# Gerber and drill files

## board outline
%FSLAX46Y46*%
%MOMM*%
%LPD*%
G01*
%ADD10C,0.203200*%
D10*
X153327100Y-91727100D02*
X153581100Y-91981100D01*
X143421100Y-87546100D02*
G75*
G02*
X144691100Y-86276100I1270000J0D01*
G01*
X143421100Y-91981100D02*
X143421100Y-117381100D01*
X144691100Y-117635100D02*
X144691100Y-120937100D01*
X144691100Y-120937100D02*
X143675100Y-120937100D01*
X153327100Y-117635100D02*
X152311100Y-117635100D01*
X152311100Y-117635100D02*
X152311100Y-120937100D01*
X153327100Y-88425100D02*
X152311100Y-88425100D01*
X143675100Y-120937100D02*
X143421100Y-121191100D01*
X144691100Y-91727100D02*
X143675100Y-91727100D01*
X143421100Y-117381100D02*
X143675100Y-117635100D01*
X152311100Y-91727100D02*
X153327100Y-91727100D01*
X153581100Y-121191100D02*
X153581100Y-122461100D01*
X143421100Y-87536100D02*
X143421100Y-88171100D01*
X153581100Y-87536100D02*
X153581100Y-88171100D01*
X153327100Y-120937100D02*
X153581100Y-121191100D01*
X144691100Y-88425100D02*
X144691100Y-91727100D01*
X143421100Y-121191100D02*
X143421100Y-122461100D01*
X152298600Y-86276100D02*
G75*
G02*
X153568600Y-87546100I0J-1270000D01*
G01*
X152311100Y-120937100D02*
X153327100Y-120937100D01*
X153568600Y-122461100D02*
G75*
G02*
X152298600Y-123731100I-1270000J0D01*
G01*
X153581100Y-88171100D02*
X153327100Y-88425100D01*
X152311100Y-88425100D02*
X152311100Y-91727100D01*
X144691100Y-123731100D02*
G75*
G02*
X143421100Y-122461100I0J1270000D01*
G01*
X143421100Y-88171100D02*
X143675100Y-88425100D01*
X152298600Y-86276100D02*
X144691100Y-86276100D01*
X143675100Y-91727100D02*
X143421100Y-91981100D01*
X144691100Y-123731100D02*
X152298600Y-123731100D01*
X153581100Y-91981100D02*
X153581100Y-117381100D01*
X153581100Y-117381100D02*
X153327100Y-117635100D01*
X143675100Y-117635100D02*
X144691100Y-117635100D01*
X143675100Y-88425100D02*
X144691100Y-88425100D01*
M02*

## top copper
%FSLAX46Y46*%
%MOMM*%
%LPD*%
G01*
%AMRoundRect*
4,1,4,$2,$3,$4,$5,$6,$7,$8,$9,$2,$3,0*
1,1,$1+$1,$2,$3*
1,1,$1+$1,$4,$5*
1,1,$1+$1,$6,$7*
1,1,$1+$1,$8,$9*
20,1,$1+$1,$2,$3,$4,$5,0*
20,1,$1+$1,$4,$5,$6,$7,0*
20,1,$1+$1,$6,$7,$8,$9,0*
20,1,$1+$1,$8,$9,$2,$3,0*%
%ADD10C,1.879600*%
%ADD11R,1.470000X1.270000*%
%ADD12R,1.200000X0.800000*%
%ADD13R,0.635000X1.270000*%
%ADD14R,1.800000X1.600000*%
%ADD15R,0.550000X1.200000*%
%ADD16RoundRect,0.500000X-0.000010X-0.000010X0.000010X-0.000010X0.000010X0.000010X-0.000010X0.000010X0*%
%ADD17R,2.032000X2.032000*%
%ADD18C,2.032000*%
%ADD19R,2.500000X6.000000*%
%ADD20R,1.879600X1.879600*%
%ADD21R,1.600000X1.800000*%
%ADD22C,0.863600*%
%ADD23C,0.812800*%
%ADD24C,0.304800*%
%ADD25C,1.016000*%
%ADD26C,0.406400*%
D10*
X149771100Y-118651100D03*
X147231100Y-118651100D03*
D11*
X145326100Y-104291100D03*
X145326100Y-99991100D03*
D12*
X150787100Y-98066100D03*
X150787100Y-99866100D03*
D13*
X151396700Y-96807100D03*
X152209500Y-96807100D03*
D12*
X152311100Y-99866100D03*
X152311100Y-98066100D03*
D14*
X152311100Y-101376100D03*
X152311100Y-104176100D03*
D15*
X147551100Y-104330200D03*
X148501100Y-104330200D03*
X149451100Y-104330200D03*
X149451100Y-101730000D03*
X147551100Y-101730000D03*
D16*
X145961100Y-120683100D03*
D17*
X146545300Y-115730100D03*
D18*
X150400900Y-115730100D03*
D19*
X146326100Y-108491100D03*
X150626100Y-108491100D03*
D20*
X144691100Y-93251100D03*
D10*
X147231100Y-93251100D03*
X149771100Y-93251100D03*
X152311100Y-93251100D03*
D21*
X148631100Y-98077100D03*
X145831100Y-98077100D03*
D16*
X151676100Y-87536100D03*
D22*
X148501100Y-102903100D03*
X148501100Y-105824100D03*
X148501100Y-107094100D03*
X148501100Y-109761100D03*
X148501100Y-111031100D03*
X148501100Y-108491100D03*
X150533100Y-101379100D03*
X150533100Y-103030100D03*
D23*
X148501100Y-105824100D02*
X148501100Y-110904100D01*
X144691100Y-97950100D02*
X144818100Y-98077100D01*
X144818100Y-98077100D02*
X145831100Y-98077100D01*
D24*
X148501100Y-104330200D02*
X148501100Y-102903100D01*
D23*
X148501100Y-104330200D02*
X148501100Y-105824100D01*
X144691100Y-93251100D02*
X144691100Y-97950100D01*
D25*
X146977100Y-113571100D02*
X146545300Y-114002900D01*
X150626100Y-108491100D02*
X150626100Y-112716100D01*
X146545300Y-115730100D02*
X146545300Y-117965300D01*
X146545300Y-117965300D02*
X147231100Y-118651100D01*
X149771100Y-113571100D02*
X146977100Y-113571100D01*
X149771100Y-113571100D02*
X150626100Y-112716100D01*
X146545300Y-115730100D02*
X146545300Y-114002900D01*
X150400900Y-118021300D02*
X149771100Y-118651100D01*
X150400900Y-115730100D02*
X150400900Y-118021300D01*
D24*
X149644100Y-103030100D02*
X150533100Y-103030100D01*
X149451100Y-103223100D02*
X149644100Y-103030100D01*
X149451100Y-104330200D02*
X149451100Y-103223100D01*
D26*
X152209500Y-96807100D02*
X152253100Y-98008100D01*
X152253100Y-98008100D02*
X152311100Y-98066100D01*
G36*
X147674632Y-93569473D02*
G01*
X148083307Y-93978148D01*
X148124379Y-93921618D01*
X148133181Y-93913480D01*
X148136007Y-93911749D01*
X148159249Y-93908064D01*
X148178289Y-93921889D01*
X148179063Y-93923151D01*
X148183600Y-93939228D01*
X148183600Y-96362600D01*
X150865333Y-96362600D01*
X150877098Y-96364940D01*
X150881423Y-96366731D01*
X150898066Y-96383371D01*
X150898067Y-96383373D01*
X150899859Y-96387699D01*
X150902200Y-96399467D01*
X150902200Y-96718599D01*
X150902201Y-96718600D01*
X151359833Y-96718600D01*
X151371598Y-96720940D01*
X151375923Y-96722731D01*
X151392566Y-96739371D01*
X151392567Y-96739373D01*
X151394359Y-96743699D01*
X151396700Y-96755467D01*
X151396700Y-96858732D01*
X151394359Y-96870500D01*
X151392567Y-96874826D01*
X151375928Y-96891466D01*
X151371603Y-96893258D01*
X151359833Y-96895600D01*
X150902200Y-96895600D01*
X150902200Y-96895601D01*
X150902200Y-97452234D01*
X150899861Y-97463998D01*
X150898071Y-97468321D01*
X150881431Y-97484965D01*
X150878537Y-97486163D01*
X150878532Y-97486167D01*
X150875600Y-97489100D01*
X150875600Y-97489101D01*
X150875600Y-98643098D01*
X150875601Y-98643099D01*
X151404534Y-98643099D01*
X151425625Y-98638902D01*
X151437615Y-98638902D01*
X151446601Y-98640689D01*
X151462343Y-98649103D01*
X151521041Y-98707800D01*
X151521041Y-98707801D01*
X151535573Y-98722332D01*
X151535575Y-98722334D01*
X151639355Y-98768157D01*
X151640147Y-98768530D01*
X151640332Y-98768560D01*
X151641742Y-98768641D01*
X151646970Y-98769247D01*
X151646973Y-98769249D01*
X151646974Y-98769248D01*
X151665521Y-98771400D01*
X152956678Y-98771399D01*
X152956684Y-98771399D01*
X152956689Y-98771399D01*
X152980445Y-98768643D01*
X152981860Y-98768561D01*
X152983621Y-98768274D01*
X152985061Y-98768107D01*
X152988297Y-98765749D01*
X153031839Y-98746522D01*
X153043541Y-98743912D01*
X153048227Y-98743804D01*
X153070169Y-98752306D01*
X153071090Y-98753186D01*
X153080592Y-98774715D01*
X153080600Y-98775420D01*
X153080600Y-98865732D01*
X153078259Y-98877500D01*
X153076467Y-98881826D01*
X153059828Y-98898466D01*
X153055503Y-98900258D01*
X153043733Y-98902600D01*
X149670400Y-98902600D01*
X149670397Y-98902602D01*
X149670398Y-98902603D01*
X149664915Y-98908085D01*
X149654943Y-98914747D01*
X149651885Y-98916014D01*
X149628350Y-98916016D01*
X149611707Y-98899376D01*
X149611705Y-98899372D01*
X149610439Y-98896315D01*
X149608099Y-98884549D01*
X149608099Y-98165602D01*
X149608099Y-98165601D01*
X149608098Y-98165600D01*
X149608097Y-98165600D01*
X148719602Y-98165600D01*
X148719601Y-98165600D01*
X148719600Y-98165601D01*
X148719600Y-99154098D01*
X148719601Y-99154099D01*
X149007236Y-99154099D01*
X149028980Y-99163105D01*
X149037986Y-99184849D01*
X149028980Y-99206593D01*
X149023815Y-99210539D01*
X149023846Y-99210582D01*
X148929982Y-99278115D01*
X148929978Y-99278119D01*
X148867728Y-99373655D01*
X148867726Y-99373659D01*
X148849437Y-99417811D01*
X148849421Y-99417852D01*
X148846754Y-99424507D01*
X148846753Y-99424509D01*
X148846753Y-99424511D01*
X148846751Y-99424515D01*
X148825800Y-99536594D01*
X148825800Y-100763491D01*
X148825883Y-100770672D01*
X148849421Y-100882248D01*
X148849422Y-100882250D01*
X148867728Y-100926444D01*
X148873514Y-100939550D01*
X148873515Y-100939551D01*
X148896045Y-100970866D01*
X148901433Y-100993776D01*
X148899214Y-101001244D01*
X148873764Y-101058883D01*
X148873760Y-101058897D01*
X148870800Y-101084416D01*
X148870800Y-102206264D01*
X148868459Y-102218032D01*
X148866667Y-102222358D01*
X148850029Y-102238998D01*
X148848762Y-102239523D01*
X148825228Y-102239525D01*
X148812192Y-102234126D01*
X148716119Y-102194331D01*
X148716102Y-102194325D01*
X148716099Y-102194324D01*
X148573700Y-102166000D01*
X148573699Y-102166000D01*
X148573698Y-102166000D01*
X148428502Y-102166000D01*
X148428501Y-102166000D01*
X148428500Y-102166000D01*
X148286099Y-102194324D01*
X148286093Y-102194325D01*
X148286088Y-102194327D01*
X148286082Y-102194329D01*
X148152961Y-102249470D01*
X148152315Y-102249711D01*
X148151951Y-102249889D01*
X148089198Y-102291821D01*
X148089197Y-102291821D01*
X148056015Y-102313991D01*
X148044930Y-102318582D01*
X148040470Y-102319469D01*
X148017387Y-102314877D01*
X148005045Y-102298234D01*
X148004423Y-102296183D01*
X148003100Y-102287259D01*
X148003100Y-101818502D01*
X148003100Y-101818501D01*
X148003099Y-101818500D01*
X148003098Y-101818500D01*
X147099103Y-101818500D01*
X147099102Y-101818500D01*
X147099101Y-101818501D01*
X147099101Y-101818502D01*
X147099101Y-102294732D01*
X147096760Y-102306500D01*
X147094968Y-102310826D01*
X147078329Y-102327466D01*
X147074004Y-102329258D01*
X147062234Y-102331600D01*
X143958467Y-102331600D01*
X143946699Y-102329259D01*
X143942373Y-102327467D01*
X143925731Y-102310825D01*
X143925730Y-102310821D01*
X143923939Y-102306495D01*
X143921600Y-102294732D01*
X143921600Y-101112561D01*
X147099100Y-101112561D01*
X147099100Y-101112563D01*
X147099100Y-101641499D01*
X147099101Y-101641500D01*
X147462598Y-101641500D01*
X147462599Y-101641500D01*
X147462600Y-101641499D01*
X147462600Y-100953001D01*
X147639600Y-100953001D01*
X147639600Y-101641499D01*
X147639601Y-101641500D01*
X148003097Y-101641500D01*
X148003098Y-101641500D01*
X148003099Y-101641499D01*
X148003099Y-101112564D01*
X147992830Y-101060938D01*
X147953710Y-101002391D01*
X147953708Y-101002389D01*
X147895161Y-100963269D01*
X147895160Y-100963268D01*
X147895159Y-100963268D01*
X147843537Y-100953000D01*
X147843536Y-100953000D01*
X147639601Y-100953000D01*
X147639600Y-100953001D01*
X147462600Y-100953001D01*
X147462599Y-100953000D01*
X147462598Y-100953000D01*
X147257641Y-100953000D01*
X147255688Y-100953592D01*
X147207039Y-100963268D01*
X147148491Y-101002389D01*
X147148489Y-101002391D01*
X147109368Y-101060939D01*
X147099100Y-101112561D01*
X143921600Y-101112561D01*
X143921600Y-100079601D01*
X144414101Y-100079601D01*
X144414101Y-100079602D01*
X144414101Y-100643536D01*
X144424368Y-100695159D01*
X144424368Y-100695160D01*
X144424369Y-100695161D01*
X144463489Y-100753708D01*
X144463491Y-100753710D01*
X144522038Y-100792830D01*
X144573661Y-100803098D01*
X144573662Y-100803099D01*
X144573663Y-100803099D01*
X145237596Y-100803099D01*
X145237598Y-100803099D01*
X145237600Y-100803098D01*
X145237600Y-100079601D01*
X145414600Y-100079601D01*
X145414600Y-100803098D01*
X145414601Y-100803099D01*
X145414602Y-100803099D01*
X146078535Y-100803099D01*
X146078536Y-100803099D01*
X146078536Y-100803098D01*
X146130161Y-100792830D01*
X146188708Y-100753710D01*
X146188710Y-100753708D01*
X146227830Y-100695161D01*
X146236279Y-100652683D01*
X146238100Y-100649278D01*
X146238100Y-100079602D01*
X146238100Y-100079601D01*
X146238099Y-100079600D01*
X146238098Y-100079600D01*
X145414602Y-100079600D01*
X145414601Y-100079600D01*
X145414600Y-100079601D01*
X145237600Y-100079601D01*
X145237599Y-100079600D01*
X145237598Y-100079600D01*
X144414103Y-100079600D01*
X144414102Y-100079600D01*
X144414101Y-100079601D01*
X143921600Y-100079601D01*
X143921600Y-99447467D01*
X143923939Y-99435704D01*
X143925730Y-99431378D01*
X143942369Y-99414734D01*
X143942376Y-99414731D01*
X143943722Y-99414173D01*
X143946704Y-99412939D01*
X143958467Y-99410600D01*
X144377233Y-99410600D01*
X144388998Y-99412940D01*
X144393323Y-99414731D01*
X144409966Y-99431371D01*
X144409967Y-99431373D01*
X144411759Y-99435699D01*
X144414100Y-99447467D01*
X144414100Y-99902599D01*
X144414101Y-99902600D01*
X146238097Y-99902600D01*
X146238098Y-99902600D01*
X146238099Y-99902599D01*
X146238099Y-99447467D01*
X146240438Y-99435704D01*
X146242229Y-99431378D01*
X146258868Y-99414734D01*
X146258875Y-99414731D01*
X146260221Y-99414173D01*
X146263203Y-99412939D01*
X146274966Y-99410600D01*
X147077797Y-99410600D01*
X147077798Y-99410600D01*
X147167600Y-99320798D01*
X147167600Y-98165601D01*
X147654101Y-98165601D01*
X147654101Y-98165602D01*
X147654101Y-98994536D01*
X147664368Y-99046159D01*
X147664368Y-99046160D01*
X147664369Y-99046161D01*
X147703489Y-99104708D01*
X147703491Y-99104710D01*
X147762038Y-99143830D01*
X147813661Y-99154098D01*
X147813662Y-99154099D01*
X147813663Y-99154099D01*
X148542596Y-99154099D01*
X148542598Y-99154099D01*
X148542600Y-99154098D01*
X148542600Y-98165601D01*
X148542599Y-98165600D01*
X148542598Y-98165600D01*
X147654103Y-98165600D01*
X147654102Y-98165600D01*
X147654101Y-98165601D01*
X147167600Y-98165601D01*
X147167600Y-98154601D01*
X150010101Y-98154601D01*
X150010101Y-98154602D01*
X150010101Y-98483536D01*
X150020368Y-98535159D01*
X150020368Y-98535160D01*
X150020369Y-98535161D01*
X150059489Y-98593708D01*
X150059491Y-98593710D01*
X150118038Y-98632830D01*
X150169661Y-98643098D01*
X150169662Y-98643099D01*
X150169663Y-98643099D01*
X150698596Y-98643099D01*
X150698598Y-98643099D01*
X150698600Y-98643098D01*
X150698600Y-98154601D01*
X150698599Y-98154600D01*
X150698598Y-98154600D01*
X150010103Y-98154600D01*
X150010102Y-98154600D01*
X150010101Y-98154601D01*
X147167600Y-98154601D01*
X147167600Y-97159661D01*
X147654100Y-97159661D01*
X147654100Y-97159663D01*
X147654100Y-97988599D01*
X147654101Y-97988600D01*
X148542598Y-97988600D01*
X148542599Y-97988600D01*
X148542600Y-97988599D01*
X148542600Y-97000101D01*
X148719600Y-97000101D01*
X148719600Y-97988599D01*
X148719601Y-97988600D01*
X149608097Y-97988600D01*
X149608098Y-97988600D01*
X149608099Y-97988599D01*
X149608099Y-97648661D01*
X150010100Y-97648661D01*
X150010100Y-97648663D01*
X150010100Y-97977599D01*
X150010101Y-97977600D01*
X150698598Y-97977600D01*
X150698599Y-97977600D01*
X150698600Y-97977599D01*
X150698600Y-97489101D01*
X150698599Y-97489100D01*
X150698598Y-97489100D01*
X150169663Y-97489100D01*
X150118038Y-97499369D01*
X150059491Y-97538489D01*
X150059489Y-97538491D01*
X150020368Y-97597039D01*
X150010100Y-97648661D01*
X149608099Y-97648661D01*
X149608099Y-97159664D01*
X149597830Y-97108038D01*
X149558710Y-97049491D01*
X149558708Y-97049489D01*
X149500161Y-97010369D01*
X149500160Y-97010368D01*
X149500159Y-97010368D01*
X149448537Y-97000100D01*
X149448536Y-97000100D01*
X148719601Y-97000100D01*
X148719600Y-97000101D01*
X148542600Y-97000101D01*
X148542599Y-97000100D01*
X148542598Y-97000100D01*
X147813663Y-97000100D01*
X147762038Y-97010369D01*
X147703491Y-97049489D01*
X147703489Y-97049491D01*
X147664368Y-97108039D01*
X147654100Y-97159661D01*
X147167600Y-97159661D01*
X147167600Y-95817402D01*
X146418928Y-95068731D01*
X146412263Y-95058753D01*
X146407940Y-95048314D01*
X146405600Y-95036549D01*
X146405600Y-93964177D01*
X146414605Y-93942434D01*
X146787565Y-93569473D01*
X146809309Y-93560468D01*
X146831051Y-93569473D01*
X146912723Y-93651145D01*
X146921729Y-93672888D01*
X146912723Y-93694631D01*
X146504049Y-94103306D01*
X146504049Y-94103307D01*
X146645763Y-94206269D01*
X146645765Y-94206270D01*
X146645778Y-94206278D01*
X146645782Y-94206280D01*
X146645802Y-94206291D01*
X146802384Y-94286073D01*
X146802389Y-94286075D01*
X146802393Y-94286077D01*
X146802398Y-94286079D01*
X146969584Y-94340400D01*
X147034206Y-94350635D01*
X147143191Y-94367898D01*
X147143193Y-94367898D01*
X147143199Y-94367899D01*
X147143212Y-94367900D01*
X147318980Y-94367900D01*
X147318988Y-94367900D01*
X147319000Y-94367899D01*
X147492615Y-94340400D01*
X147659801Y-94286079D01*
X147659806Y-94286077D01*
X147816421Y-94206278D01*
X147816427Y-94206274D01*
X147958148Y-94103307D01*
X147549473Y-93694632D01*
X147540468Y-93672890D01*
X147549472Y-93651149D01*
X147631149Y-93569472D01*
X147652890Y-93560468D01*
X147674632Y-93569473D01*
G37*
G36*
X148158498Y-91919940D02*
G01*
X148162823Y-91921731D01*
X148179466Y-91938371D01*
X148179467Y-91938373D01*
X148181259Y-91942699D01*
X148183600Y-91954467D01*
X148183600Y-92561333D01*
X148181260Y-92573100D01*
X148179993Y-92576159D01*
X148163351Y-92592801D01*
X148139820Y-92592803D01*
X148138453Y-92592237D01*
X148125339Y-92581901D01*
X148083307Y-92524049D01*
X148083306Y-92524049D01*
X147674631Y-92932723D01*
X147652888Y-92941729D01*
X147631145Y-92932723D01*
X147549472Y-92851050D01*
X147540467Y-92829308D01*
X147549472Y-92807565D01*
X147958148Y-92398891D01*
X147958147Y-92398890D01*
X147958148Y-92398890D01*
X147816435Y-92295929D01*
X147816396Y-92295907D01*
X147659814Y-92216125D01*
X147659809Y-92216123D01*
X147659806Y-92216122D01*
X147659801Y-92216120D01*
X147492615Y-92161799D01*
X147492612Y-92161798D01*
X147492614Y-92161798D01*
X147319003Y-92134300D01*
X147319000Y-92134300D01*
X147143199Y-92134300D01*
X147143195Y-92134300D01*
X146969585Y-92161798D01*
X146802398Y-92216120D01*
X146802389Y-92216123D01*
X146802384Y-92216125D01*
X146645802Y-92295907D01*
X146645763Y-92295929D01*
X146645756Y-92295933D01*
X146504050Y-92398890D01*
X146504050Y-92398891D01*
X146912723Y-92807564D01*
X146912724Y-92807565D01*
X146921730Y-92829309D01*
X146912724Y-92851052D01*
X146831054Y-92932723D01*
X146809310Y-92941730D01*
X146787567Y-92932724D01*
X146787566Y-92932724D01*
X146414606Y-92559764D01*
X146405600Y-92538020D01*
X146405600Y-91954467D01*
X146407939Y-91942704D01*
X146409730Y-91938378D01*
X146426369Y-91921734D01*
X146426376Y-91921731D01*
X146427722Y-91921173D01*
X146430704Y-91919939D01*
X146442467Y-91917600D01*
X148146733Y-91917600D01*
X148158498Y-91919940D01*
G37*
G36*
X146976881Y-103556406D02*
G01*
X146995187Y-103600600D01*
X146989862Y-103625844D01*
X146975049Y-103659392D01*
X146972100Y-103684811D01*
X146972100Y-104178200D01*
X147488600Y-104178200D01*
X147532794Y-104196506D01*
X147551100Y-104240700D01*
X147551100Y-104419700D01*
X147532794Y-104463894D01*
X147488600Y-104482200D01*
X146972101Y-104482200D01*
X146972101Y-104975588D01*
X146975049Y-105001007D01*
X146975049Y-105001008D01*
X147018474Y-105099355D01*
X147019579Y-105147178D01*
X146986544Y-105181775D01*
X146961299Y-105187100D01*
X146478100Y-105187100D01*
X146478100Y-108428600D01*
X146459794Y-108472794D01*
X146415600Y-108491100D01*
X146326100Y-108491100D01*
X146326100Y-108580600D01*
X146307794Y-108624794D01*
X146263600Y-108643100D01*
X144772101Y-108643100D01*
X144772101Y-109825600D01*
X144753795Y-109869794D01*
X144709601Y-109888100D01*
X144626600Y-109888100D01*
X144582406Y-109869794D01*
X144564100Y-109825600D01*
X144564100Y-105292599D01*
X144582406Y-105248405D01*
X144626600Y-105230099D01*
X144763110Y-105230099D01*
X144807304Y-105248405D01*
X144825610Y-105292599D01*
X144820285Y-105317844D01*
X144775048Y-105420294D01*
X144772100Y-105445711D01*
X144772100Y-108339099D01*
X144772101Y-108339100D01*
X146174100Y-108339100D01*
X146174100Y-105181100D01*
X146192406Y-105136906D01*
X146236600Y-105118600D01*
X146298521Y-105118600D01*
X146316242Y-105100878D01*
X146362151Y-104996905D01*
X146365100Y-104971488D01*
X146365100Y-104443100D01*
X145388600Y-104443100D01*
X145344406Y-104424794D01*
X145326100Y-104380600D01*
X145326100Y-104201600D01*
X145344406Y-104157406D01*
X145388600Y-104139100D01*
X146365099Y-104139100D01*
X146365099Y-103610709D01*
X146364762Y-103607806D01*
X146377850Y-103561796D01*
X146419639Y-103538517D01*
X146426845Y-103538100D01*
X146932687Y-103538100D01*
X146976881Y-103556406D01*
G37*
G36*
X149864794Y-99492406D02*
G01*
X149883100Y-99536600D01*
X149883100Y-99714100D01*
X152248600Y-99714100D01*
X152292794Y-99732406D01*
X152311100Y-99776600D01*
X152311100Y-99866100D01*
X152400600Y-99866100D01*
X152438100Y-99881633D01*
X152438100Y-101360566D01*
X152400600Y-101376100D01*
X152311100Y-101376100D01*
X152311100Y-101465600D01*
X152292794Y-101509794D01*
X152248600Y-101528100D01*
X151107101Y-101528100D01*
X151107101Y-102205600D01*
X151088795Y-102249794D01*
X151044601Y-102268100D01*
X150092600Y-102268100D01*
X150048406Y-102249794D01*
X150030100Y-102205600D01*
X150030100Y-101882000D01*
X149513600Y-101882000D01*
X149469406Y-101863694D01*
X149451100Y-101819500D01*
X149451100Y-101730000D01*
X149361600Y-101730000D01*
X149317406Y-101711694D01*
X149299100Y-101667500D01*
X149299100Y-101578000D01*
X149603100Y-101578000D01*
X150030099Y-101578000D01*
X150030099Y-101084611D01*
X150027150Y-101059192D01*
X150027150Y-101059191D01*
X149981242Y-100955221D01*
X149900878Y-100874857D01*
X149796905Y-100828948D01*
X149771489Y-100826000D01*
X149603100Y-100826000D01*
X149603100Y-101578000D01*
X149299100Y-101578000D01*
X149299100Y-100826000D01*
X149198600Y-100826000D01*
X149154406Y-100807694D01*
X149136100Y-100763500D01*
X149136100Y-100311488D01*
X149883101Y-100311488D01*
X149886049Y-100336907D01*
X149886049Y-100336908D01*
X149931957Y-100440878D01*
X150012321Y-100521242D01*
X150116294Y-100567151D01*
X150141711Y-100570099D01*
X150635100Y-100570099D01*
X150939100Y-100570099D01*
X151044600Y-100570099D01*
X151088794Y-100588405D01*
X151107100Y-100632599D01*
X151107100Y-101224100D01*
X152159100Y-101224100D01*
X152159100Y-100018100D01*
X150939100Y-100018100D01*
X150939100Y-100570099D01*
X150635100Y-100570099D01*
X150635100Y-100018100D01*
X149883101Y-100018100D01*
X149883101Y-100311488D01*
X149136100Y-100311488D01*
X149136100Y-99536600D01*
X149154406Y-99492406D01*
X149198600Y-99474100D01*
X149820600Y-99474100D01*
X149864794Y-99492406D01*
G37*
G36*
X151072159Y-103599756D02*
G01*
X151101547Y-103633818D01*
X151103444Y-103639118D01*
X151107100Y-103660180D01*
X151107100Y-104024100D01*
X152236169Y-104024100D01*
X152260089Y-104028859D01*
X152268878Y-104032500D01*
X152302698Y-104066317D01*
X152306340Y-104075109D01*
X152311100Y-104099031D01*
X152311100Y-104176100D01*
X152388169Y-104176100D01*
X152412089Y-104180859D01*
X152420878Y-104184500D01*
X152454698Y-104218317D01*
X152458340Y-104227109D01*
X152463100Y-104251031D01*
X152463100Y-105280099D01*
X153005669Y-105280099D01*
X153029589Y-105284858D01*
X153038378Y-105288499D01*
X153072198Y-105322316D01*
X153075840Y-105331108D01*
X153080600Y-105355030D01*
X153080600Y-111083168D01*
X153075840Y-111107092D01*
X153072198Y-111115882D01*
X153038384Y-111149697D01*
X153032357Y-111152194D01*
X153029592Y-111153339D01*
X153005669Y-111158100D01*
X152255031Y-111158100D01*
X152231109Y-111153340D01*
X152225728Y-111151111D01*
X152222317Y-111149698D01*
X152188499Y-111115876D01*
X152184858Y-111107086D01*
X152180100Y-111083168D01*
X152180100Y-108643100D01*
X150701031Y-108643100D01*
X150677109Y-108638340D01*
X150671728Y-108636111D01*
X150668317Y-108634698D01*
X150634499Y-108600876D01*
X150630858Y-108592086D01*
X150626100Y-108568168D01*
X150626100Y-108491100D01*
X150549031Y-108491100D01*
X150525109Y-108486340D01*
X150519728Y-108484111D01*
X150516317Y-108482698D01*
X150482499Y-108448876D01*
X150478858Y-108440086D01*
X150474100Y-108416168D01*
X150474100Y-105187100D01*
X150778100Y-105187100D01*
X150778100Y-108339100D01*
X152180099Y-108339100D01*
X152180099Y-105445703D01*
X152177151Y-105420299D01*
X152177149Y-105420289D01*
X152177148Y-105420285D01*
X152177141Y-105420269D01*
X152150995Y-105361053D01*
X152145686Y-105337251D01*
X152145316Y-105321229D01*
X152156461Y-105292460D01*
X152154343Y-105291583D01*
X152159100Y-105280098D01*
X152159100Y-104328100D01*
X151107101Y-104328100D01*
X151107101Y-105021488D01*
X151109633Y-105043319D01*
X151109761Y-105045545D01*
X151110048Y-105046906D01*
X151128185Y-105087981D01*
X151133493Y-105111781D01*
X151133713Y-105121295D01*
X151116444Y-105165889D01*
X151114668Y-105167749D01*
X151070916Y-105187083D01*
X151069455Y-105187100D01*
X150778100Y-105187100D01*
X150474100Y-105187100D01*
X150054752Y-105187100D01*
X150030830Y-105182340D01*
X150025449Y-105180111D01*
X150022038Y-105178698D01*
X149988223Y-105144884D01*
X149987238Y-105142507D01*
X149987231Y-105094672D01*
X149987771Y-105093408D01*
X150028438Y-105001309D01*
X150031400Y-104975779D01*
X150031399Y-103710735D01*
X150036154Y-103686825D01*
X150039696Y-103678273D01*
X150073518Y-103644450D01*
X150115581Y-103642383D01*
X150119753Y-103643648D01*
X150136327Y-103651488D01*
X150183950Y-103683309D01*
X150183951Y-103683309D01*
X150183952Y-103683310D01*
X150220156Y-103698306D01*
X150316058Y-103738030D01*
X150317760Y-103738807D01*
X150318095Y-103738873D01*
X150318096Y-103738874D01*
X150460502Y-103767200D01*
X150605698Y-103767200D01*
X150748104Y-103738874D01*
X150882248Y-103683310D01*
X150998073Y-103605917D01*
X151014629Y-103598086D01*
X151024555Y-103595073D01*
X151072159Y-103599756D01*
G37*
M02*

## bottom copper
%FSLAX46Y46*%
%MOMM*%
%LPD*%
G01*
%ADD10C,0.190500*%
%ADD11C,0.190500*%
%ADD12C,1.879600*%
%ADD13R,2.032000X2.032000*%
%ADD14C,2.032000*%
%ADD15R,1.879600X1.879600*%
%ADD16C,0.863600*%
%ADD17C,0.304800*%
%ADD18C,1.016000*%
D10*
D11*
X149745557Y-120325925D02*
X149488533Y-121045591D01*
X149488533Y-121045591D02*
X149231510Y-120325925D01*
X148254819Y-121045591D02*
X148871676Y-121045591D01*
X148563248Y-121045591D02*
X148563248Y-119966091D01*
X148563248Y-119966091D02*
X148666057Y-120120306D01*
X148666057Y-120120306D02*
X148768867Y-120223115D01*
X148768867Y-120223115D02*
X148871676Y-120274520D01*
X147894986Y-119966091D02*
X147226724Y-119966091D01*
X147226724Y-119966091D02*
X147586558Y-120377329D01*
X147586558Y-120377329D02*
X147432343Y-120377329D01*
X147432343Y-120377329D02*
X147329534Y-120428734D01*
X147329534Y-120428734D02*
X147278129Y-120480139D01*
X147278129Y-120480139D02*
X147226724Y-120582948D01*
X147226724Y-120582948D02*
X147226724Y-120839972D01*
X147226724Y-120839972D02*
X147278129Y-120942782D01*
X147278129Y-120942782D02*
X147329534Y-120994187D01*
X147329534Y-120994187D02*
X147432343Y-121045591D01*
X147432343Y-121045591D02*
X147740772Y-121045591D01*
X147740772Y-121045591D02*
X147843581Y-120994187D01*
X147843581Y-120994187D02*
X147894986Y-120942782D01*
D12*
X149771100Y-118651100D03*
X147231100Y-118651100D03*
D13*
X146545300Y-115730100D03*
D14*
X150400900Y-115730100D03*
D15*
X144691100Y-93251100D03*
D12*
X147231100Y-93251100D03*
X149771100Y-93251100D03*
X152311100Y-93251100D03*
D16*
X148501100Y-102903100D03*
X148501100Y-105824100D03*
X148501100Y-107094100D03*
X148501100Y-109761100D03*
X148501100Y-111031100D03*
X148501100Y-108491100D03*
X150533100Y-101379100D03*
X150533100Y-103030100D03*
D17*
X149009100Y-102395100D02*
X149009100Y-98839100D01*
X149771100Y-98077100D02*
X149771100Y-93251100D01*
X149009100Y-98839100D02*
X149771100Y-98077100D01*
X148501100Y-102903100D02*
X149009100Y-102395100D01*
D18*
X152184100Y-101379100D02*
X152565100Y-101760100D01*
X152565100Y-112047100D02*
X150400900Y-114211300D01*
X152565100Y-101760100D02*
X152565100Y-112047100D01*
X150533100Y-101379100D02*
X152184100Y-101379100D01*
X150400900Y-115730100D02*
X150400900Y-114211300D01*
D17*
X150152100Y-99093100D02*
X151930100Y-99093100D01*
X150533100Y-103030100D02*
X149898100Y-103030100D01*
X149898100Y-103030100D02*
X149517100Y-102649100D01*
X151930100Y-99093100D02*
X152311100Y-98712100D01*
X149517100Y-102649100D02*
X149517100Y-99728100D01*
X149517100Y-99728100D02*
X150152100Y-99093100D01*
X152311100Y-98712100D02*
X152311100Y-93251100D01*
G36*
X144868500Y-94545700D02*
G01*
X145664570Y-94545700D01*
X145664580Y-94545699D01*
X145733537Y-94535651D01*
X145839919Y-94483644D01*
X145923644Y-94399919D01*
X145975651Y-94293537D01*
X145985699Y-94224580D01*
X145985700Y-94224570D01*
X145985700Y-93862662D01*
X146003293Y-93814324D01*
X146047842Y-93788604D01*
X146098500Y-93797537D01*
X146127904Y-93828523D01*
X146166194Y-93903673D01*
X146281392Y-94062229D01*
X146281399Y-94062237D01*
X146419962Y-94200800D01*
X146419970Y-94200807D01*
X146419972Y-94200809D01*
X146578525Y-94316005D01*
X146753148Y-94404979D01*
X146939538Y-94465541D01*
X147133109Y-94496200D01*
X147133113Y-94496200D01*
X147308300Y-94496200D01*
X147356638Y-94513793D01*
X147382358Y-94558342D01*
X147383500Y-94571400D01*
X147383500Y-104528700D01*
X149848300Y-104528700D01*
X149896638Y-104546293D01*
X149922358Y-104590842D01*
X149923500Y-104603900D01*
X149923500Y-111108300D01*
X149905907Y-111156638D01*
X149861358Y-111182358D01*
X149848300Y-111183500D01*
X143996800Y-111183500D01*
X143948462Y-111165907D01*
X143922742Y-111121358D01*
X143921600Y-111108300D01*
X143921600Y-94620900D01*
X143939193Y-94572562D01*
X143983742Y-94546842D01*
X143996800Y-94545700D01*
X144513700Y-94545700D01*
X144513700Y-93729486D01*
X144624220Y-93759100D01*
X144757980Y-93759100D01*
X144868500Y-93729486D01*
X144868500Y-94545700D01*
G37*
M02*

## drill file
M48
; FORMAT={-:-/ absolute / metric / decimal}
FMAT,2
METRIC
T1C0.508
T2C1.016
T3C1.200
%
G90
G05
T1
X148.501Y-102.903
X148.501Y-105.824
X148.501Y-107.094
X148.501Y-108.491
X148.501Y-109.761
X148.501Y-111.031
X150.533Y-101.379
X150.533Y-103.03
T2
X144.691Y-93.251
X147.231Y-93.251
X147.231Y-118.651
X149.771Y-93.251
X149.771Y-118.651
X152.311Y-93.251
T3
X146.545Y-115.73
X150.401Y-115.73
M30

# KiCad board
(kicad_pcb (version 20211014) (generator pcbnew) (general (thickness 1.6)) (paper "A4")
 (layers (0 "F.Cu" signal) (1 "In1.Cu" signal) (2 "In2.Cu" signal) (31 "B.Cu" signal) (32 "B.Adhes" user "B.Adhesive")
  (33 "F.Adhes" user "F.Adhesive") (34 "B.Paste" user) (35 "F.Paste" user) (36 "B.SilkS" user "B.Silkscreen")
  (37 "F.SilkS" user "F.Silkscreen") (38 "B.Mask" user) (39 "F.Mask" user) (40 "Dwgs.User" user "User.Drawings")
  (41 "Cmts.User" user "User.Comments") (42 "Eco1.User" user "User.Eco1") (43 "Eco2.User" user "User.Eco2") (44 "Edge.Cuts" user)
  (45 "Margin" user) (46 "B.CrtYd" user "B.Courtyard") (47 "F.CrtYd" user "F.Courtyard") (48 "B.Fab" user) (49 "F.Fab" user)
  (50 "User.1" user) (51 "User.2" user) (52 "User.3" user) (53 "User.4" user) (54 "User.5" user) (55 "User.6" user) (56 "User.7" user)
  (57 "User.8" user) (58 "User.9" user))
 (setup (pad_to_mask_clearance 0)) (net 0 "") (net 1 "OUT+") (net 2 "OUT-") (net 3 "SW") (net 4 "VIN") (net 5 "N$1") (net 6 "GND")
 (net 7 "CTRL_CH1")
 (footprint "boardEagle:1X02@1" (layer "F.Cu") (at 149.7711 118.6511 180)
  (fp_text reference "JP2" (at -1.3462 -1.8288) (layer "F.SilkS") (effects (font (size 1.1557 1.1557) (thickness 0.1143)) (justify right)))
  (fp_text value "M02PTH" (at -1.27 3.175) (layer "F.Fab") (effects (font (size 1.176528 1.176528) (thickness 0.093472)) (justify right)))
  (pad "1" thru_hole circle (at 0 0 270) (size 1.8796 1.8796) (drill 1.016) (layers *.Cu *.Mask) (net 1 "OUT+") (solder_mask_margin 0.1016))
  (pad "2" thru_hole circle (at 2.54 0 270) (size 1.8796 1.8796) (drill 1.016) (layers *.Cu *.Mask) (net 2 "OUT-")
   (solder_mask_margin 0.1016)))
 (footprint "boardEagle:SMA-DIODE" (layer "F.Cu") (at 145.3261 102.1411 90)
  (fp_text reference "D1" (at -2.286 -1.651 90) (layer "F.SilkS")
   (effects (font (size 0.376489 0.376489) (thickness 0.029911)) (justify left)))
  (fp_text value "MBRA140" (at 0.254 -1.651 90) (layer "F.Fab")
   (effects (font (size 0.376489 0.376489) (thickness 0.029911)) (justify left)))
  (pad "A" smd rect (at -2.15 0 270) (size 1.27 1.47) (layers "F.Cu" "F.Paste" "F.Mask") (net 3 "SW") (solder_mask_margin 0.1016))
  (pad "C" smd rect (at 2.15 0 90) (size 1.27 1.47) (layers "F.Cu" "F.Paste" "F.Mask") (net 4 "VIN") (solder_mask_margin 0.1016)))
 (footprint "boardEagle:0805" (layer "F.Cu") (at 150.7871 98.9661 -90)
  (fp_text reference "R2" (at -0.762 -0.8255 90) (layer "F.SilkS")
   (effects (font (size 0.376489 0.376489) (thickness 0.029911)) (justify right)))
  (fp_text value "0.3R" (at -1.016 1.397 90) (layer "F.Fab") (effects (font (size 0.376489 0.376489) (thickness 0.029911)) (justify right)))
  (pad "1" smd rect (at -0.9 0 270) (size 0.8 1.2) (layers "F.Cu" "F.Paste" "F.Mask") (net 4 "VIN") (solder_mask_margin 0.1016))
  (pad "2" smd rect (at 0.9 0 270) (size 0.8 1.2) (layers "F.Cu" "F.Paste" "F.Mask") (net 1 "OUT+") (solder_mask_margin 0.1016)))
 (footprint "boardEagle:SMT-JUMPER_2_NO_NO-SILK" (layer "F.Cu") (at 151.8031 96.8071)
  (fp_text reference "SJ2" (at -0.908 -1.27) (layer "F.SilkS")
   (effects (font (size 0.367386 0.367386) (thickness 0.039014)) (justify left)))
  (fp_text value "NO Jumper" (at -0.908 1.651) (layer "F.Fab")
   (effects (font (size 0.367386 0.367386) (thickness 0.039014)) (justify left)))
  (pad "1" smd rect (at -0.4064 0) (size 0.635 1.27) (layers "F.Cu" "F.Mask") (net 4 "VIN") (solder_mask_margin 0.1016))
  (pad "2" smd rect (at 0.4064 0) (size 0.635 1.27) (layers "F.Cu" "F.Mask") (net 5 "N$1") (solder_mask_margin 0.1016)))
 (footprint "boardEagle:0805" (layer "F.Cu") (at 152.3111 98.9661 90)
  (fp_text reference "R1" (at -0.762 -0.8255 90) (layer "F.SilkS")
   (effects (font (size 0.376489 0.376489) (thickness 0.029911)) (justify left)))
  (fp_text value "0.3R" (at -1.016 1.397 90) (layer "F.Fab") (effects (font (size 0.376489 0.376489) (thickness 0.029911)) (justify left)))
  (pad "1" smd rect (at -0.9 0 90) (size 0.8 1.2) (layers "F.Cu" "F.Paste" "F.Mask") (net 1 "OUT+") (solder_mask_margin 0.1016))
  (pad "2" smd rect (at 0.9 0 90) (size 0.8 1.2) (layers "F.Cu" "F.Paste" "F.Mask") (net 5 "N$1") (solder_mask_margin 0.1016)))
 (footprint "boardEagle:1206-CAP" (layer "F.Cu") (at 152.3111 102.7761 -90)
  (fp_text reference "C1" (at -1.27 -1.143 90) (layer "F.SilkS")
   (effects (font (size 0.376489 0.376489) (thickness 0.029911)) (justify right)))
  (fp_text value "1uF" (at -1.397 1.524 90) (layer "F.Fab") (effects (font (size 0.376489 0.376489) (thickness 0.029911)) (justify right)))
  (pad "1" smd rect (at -1.4 0 270) (size 1.6 1.8) (layers "F.Cu" "F.Paste" "F.Mask") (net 1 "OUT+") (solder_mask_margin 0.1016))
  (pad "2" smd rect (at 1.4 0 270) (size 1.6 1.8) (layers "F.Cu" "F.Paste" "F.Mask") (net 2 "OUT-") (solder_mask_margin 0.1016)))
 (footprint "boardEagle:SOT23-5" (layer "F.Cu") (at 148.5011 103.0301)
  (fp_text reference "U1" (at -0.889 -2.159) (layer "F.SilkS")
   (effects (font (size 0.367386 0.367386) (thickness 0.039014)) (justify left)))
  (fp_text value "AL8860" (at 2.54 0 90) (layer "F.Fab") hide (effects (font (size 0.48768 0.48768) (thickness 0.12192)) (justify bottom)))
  (pad "1" smd rect (at -0.95 1.3001) (size 0.55 1.2) (layers "F.Cu" "F.Paste" "F.Mask") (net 3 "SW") (solder_mask_margin 0.1016))
  (pad "2" smd rect (at 0 1.3001) (size 0.55 1.2) (layers "F.Cu" "F.Paste" "F.Mask") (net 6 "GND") (solder_mask_margin 0.1016))
  (pad "3" smd rect (at 0.95 1.3001) (size 0.55 1.2) (layers "F.Cu" "F.Paste" "F.Mask") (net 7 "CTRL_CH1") (solder_mask_margin 0.1016))
  (pad "4" smd rect (at 0.95 -1.3001) (size 0.55 1.2) (layers "F.Cu" "F.Paste" "F.Mask") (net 1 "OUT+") (solder_mask_margin 0.1016))
  (pad "5" smd rect (at -0.95 -1.3001) (size 0.55 1.2) (layers "F.Cu" "F.Paste" "F.Mask") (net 4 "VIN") (solder_mask_margin 0.1016)))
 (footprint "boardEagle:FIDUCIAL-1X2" (layer "F.Cu") (at 145.9611 120.6831)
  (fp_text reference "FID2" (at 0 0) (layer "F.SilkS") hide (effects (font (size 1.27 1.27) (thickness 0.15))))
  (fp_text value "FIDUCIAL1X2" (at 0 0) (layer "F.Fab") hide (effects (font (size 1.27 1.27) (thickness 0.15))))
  (pad "1" smd roundrect (at 0 0) (size 1 1) (layers "F.Cu" "F.Mask") (roundrect_rratio 0.5) (solder_mask_margin 0.1016)))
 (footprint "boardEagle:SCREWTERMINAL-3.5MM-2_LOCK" (layer "F.Cu") (at 146.7231 115.7301)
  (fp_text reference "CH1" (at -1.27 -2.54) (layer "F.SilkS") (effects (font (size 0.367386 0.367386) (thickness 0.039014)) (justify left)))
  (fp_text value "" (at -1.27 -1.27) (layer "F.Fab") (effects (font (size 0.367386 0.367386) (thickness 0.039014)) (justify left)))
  (pad "1" thru_hole rect (at -0.1778 0) (size 2.032 2.032) (drill 1.2) (layers *.Cu *.Mask) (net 2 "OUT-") (solder_mask_margin 0.1016))
  (pad "2" thru_hole circle (at 3.6778 0) (size 2.032 2.032) (drill 1.2) (layers *.Cu *.Mask) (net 1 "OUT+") (solder_mask_margin 0.1016)))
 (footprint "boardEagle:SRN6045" (layer "F.Cu") (at 148.5011 108.4911)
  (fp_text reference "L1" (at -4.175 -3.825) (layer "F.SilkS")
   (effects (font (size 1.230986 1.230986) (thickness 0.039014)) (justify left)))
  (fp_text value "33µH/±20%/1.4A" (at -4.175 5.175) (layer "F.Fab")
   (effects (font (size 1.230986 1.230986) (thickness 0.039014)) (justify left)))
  (pad "1" smd rect (at -2.175 0 90) (size 6 2.5) (layers "F.Cu" "F.Paste" "F.Mask") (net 3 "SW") (solder_mask_margin 0.1016))
  (pad "2" smd rect (at 2.125 0 90) (size 6 2.5) (layers "F.Cu" "F.Paste" "F.Mask") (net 2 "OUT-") (solder_mask_margin 0.1016)))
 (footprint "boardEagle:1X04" (layer "F.Cu") (at 144.6911 93.2511)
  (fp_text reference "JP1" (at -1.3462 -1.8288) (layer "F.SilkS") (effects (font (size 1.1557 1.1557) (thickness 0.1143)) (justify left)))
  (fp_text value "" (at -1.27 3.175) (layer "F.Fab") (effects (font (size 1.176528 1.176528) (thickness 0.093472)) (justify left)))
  (pad "1" thru_hole rect (at 0 0 90) (size 1.8796 1.8796) (drill 1.016) (layers *.Cu *.Mask) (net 6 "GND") (solder_mask_margin 0.1016))
  (pad "2" thru_hole circle (at 2.54 0 90) (size 1.8796 1.8796) (drill 1.016) (layers *.Cu *.Mask) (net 4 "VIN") (solder_mask_margin 0.1016))
  (pad "3" thru_hole circle (at 5.08 0 90) (size 1.8796 1.8796) (drill 1.016) (layers *.Cu *.Mask) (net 6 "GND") (solder_mask_margin 0.1016))
  (pad "4" thru_hole circle (at 7.62 0 90) (size 1.8796 1.8796) (drill 1.016) (layers *.Cu *.Mask) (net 7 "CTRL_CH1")
   (solder_mask_margin 0.1016)))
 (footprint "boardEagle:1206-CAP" (layer "F.Cu") (at 147.2311 98.0771 180)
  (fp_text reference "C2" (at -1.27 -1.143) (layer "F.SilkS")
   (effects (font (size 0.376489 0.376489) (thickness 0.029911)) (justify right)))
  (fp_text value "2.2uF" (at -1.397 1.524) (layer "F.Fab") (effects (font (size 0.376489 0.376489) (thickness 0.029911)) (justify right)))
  (pad "1" smd rect (at -1.4 0 180) (size 1.6 1.8) (layers "F.Cu" "F.Paste" "F.Mask") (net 4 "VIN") (solder_mask_margin 0.1016))
  (pad "2" smd rect (at 1.4 0 180) (size 1.6 1.8) (layers "F.Cu" "F.Paste" "F.Mask") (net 6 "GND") (solder_mask_margin 0.1016)))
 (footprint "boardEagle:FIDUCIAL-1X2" (layer "F.Cu") (at 151.6761 87.5361)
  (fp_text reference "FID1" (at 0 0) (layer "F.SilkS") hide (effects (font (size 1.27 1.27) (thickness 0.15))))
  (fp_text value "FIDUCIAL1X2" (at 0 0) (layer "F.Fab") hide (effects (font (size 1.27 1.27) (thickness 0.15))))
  (pad "1" smd roundrect (at 0 0) (size 1 1) (layers "F.Cu" "F.Mask") (roundrect_rratio 0.5) (solder_mask_margin 0.1016)))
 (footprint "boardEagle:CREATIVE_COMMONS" (layer "F.Cu") (at 154.8511 145.3211)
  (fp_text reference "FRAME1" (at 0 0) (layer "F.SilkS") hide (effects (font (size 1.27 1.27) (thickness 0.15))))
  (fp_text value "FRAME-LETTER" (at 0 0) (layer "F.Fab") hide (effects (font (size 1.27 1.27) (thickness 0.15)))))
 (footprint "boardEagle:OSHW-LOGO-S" (layer "B.Cu") (at 145.4531 98.7121 -90)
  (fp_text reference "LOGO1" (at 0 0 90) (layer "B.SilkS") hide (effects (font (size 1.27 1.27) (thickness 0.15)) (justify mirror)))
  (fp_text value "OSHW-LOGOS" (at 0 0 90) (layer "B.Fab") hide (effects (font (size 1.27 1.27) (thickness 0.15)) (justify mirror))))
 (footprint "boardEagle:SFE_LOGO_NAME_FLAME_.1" (layer "B.Cu") (at 153.2001 100.6171 -90)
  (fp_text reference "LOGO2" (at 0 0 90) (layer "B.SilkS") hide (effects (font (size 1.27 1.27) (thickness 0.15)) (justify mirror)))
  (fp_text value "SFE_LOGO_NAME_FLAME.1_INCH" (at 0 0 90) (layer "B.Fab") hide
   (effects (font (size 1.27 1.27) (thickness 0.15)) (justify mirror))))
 (gr_line (start 153.3271 91.7271) (end 153.5811 91.9811) (layer "Edge.Cuts") (width 0.2032))
 (gr_arc (start 143.4211 87.5461) (mid 143.793074 86.648074) (end 144.6911 86.2761) (layer "Edge.Cuts") (width 0.2032))
 (gr_line (start 143.4211 91.9811) (end 143.4211 117.3811) (layer "Edge.Cuts") (width 0.2032))
 (gr_line (start 144.6911 117.6351) (end 144.6911 120.9371) (layer "Edge.Cuts") (width 0.2032))
 (gr_line (start 144.6911 120.9371) (end 143.6751 120.9371) (layer "Edge.Cuts") (width 0.2032))
 (gr_line (start 153.3271 117.6351) (end 152.3111 117.6351) (layer "Edge.Cuts") (width 0.2032))
 (gr_line (start 152.3111 117.6351) (end 152.3111 120.9371) (layer "Edge.Cuts") (width 0.2032))
 (gr_line (start 153.3271 88.4251) (end 152.3111 88.4251) (layer "Edge.Cuts") (width 0.2032))
 (gr_line (start 143.6751 120.9371) (end 143.4211 121.1911) (layer "Edge.Cuts") (width 0.2032))
 (gr_line (start 144.6911 91.7271) (end 143.6751 91.7271) (layer "Edge.Cuts") (width 0.2032))
 (gr_line (start 143.4211 117.3811) (end 143.6751 117.6351) (layer "Edge.Cuts") (width 0.2032))
 (gr_line (start 152.3111 91.7271) (end 153.3271 91.7271) (layer "Edge.Cuts") (width 0.2032))
 (gr_line (start 153.5811 121.1911) (end 153.5811 122.4611) (layer "Edge.Cuts") (width 0.2032))
 (gr_line (start 143.4211 87.5361) (end 143.4211 88.1711) (layer "Edge.Cuts") (width 0.2032))
 (gr_line (start 153.5811 87.5361) (end 153.5811 88.1711) (layer "Edge.Cuts") (width 0.2032))
 (gr_line (start 153.3271 120.9371) (end 153.5811 121.1911) (layer "Edge.Cuts") (width 0.2032))
 (gr_line (start 144.6911 88.4251) (end 144.6911 91.7271) (layer "Edge.Cuts") (width 0.2032))
 (gr_line (start 143.4211 121.1911) (end 143.4211 122.4611) (layer "Edge.Cuts") (width 0.2032))
 (gr_arc (start 152.2986 86.2761) (mid 153.196626 86.648074) (end 153.5686 87.5461) (layer "Edge.Cuts") (width 0.2032))
 (gr_line (start 152.3111 120.9371) (end 153.3271 120.9371) (layer "Edge.Cuts") (width 0.2032))
 (gr_arc (start 153.5686 122.4611) (mid 153.196626 123.359126) (end 152.2986 123.7311) (layer "Edge.Cuts") (width 0.2032))
 (gr_line (start 153.5811 88.1711) (end 153.3271 88.4251) (layer "Edge.Cuts") (width 0.2032))
 (gr_line (start 152.3111 88.4251) (end 152.3111 91.7271) (layer "Edge.Cuts") (width 0.2032))
 (gr_arc (start 144.6911 123.7311) (mid 143.793074 123.359126) (end 143.4211 122.4611) (layer "Edge.Cuts") (width 0.2032))
 (gr_line (start 143.4211 88.1711) (end 143.6751 88.4251) (layer "Edge.Cuts") (width 0.2032))
 (gr_line (start 152.2986 86.2761) (end 144.6911 86.2761) (layer "Edge.Cuts") (width 0.2032))
 (gr_line (start 143.6751 91.7271) (end 143.4211 91.9811) (layer "Edge.Cuts") (width 0.2032))
 (gr_line (start 144.6911 123.7311) (end 152.2986 123.7311) (layer "Edge.Cuts") (width 0.2032))
 (gr_line (start 153.5811 91.9811) (end 153.5811 117.3811) (layer "Edge.Cuts") (width 0.2032))
 (gr_line (start 153.5811 117.3811) (end 153.3271 117.6351) (layer "Edge.Cuts") (width 0.2032))
 (gr_line (start 143.6751 117.6351) (end 144.6911 117.6351) (layer "Edge.Cuts") (width 0.2032))
 (gr_line (start 143.6751 88.4251) (end 144.6911 88.4251) (layer "Edge.Cuts") (width 0.2032))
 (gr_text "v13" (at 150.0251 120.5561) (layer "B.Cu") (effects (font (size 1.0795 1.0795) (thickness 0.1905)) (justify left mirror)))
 (segment (start 148.5011 105.8241) (end 148.5011 110.9041) (width 0.8128) (layer "F.Cu") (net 6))
 (segment (start 144.6911 97.9501) (end 144.8181 98.0771) (width 0.8128) (layer "F.Cu") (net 6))
 (segment (start 144.8181 98.0771) (end 145.8311 98.0771) (width 0.8128) (layer "F.Cu") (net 6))
 (segment (start 148.5011 104.3302) (end 148.5011 102.9031) (width 0.3048) (layer "F.Cu") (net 6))
 (segment (start 148.5011 104.3302) (end 148.5011 105.8241) (width 0.8128) (layer "F.Cu") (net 6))
 (segment (start 144.6911 93.2511) (end 144.6911 97.9501) (width 0.8128) (layer "F.Cu") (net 6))
 (via (at 148.5011 102.9031) (size 0.8636) (drill 0.508) (layers "F.Cu" "B.Cu") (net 6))
 (via (at 148.5011 105.8241) (size 0.8636) (drill 0.508) (layers "F.Cu" "B.Cu") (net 6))
 (via (at 148.5011 107.0941) (size 0.8636) (drill 0.508) (layers "F.Cu" "B.Cu") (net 6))
 (via (at 148.5011 109.7611) (size 0.8636) (drill 0.508) (layers "F.Cu" "B.Cu") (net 6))
 (via (at 148.5011 111.0311) (size 0.8636) (drill 0.508) (layers "F.Cu" "B.Cu") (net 6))
 (via (at 148.5011 108.4911) (size 0.8636) (drill 0.508) (layers "F.Cu" "B.Cu") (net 6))
 (segment (start 149.0091 102.3951) (end 149.0091 98.8391) (width 0.3048) (layer "B.Cu") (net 6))
 (segment (start 149.7711 98.0771) (end 149.7711 93.2511) (width 0.3048) (layer "B.Cu") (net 6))
 (segment (start 149.0091 98.8391) (end 149.7711 98.0771) (width 0.3048) (layer "B.Cu") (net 6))
 (segment (start 148.5011 102.9031) (end 149.0091 102.3951) (width 0.3048) (layer "B.Cu") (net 6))
 (segment (start 146.9771 113.5711) (end 146.5453 114.0029) (width 1.016) (layer "F.Cu") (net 2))
 (segment (start 150.6261 108.4911) (end 150.6261 112.7161) (width 1.016) (layer "F.Cu") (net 2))
 (segment (start 146.5453 115.7301) (end 146.5453 117.9653) (width 1.016) (layer "F.Cu") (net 2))
 (segment (start 146.5453 117.9653) (end 147.2311 118.6511) (width 1.016) (layer "F.Cu") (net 2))
 (segment (start 149.7711 113.5711) (end 146.9771 113.5711) (width 1.016) (layer "F.Cu") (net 2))
 (segment (start 149.7711 113.5711) (end 150.6261 112.7161) (width 1.016) (layer "F.Cu") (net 2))
 (segment (start 146.5453 115.7301) (end 146.5453 114.0029) (width 1.016) (layer "F.Cu") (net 2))
 (segment (start 150.4009 118.0213) (end 149.7711 118.6511) (width 1.016) (layer "F.Cu") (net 1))
 (segment (start 150.4009 115.7301) (end 150.4009 118.0213) (width 1.016) (layer "F.Cu") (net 1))
 (via (at 150.5331 101.3791) (size 0.8636) (drill 0.508) (layers "F.Cu" "B.Cu") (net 1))
 (segment (start 152.1841 101.3791) (end 152.5651 101.7601) (width 1.016) (layer "B.Cu") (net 1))
 (segment (start 152.5651 112.0471) (end 150.4009 114.2113) (width 1.016) (layer "B.Cu") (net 1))
 (segment (start 152.5651 101.7601) (end 152.5651 112.0471) (width 1.016) (layer "B.Cu") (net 1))
 (segment (start 150.5331 101.3791) (end 152.1841 101.3791) (width 1.016) (layer "B.Cu") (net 1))
 (segment (start 150.4009 115.7301) (end 150.4009 114.2113) (width 1.016) (layer "B.Cu") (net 1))
 (segment (start 149.6441 103.0301) (end 150.5331 103.0301) (width 0.3048) (layer "F.Cu") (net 7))
 (segment (start 149.4511 103.2231) (end 149.6441 103.0301) (width 0.3048) (layer "F.Cu") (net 7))
 (segment (start 149.4511 104.3302) (end 149.4511 103.2231) (width 0.3048) (layer "F.Cu") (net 7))
 (via (at 150.5331 103.0301) (size 0.8636) (drill 0.508) (layers "F.Cu" "B.Cu") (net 7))
 (segment (start 150.1521 99.0931) (end 151.9301 99.0931) (width 0.3048) (layer "B.Cu") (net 7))
 (segment (start 150.5331 103.0301) (end 149.8981 103.0301) (width 0.3048) (layer "B.Cu") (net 7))
 (segment (start 149.8981 103.0301) (end 149.5171 102.6491) (width 0.3048) (layer "B.Cu") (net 7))
 (segment (start 151.9301 99.0931) (end 152.3111 98.7121) (width 0.3048) (layer "B.Cu") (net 7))
 (segment (start 149.5171 102.6491) (end 149.5171 99.7281) (width 0.3048) (layer "B.Cu") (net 7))
 (segment (start 149.5171 99.7281) (end 150.1521 99.0931) (width 0.3048) (layer "B.Cu") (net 7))
 (segment (start 152.3111 98.7121) (end 152.3111 93.2511) (width 0.3048) (layer "B.Cu") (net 7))
 (segment (start 152.2095 96.8071) (end 152.2531 98.0081) (width 0.4064) (layer "F.Cu") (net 5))
 (segment (start 152.2531 98.0081) (end 152.3111 98.0661) (width 0.4064) (layer "F.Cu") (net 5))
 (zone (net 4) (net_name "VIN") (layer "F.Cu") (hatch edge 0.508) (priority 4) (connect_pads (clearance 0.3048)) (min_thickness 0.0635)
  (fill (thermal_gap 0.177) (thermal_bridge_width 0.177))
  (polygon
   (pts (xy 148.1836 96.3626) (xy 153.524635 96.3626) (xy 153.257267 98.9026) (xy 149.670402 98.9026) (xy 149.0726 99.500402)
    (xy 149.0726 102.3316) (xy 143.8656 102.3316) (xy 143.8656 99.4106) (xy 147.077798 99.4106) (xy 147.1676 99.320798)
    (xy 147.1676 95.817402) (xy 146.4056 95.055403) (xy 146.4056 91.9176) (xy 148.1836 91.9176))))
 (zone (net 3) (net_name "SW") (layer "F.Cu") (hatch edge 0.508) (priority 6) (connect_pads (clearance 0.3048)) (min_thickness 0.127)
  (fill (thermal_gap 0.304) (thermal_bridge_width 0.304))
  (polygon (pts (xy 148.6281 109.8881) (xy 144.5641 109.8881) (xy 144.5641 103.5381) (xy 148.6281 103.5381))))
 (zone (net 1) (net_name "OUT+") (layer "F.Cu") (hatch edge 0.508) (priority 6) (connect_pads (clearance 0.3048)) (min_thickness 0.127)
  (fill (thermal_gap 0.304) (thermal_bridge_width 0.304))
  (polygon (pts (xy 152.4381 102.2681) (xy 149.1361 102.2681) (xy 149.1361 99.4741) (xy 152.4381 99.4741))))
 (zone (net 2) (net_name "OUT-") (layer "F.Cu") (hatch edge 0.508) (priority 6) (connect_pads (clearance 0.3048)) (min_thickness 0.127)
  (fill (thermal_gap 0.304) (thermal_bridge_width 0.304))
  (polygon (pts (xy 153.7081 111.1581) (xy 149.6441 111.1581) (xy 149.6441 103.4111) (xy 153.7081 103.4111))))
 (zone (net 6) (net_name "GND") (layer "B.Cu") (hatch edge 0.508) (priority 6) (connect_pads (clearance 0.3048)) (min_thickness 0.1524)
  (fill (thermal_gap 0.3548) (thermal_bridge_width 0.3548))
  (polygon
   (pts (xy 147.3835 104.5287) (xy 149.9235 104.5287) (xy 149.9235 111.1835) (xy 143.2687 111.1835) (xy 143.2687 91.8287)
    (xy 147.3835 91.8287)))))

